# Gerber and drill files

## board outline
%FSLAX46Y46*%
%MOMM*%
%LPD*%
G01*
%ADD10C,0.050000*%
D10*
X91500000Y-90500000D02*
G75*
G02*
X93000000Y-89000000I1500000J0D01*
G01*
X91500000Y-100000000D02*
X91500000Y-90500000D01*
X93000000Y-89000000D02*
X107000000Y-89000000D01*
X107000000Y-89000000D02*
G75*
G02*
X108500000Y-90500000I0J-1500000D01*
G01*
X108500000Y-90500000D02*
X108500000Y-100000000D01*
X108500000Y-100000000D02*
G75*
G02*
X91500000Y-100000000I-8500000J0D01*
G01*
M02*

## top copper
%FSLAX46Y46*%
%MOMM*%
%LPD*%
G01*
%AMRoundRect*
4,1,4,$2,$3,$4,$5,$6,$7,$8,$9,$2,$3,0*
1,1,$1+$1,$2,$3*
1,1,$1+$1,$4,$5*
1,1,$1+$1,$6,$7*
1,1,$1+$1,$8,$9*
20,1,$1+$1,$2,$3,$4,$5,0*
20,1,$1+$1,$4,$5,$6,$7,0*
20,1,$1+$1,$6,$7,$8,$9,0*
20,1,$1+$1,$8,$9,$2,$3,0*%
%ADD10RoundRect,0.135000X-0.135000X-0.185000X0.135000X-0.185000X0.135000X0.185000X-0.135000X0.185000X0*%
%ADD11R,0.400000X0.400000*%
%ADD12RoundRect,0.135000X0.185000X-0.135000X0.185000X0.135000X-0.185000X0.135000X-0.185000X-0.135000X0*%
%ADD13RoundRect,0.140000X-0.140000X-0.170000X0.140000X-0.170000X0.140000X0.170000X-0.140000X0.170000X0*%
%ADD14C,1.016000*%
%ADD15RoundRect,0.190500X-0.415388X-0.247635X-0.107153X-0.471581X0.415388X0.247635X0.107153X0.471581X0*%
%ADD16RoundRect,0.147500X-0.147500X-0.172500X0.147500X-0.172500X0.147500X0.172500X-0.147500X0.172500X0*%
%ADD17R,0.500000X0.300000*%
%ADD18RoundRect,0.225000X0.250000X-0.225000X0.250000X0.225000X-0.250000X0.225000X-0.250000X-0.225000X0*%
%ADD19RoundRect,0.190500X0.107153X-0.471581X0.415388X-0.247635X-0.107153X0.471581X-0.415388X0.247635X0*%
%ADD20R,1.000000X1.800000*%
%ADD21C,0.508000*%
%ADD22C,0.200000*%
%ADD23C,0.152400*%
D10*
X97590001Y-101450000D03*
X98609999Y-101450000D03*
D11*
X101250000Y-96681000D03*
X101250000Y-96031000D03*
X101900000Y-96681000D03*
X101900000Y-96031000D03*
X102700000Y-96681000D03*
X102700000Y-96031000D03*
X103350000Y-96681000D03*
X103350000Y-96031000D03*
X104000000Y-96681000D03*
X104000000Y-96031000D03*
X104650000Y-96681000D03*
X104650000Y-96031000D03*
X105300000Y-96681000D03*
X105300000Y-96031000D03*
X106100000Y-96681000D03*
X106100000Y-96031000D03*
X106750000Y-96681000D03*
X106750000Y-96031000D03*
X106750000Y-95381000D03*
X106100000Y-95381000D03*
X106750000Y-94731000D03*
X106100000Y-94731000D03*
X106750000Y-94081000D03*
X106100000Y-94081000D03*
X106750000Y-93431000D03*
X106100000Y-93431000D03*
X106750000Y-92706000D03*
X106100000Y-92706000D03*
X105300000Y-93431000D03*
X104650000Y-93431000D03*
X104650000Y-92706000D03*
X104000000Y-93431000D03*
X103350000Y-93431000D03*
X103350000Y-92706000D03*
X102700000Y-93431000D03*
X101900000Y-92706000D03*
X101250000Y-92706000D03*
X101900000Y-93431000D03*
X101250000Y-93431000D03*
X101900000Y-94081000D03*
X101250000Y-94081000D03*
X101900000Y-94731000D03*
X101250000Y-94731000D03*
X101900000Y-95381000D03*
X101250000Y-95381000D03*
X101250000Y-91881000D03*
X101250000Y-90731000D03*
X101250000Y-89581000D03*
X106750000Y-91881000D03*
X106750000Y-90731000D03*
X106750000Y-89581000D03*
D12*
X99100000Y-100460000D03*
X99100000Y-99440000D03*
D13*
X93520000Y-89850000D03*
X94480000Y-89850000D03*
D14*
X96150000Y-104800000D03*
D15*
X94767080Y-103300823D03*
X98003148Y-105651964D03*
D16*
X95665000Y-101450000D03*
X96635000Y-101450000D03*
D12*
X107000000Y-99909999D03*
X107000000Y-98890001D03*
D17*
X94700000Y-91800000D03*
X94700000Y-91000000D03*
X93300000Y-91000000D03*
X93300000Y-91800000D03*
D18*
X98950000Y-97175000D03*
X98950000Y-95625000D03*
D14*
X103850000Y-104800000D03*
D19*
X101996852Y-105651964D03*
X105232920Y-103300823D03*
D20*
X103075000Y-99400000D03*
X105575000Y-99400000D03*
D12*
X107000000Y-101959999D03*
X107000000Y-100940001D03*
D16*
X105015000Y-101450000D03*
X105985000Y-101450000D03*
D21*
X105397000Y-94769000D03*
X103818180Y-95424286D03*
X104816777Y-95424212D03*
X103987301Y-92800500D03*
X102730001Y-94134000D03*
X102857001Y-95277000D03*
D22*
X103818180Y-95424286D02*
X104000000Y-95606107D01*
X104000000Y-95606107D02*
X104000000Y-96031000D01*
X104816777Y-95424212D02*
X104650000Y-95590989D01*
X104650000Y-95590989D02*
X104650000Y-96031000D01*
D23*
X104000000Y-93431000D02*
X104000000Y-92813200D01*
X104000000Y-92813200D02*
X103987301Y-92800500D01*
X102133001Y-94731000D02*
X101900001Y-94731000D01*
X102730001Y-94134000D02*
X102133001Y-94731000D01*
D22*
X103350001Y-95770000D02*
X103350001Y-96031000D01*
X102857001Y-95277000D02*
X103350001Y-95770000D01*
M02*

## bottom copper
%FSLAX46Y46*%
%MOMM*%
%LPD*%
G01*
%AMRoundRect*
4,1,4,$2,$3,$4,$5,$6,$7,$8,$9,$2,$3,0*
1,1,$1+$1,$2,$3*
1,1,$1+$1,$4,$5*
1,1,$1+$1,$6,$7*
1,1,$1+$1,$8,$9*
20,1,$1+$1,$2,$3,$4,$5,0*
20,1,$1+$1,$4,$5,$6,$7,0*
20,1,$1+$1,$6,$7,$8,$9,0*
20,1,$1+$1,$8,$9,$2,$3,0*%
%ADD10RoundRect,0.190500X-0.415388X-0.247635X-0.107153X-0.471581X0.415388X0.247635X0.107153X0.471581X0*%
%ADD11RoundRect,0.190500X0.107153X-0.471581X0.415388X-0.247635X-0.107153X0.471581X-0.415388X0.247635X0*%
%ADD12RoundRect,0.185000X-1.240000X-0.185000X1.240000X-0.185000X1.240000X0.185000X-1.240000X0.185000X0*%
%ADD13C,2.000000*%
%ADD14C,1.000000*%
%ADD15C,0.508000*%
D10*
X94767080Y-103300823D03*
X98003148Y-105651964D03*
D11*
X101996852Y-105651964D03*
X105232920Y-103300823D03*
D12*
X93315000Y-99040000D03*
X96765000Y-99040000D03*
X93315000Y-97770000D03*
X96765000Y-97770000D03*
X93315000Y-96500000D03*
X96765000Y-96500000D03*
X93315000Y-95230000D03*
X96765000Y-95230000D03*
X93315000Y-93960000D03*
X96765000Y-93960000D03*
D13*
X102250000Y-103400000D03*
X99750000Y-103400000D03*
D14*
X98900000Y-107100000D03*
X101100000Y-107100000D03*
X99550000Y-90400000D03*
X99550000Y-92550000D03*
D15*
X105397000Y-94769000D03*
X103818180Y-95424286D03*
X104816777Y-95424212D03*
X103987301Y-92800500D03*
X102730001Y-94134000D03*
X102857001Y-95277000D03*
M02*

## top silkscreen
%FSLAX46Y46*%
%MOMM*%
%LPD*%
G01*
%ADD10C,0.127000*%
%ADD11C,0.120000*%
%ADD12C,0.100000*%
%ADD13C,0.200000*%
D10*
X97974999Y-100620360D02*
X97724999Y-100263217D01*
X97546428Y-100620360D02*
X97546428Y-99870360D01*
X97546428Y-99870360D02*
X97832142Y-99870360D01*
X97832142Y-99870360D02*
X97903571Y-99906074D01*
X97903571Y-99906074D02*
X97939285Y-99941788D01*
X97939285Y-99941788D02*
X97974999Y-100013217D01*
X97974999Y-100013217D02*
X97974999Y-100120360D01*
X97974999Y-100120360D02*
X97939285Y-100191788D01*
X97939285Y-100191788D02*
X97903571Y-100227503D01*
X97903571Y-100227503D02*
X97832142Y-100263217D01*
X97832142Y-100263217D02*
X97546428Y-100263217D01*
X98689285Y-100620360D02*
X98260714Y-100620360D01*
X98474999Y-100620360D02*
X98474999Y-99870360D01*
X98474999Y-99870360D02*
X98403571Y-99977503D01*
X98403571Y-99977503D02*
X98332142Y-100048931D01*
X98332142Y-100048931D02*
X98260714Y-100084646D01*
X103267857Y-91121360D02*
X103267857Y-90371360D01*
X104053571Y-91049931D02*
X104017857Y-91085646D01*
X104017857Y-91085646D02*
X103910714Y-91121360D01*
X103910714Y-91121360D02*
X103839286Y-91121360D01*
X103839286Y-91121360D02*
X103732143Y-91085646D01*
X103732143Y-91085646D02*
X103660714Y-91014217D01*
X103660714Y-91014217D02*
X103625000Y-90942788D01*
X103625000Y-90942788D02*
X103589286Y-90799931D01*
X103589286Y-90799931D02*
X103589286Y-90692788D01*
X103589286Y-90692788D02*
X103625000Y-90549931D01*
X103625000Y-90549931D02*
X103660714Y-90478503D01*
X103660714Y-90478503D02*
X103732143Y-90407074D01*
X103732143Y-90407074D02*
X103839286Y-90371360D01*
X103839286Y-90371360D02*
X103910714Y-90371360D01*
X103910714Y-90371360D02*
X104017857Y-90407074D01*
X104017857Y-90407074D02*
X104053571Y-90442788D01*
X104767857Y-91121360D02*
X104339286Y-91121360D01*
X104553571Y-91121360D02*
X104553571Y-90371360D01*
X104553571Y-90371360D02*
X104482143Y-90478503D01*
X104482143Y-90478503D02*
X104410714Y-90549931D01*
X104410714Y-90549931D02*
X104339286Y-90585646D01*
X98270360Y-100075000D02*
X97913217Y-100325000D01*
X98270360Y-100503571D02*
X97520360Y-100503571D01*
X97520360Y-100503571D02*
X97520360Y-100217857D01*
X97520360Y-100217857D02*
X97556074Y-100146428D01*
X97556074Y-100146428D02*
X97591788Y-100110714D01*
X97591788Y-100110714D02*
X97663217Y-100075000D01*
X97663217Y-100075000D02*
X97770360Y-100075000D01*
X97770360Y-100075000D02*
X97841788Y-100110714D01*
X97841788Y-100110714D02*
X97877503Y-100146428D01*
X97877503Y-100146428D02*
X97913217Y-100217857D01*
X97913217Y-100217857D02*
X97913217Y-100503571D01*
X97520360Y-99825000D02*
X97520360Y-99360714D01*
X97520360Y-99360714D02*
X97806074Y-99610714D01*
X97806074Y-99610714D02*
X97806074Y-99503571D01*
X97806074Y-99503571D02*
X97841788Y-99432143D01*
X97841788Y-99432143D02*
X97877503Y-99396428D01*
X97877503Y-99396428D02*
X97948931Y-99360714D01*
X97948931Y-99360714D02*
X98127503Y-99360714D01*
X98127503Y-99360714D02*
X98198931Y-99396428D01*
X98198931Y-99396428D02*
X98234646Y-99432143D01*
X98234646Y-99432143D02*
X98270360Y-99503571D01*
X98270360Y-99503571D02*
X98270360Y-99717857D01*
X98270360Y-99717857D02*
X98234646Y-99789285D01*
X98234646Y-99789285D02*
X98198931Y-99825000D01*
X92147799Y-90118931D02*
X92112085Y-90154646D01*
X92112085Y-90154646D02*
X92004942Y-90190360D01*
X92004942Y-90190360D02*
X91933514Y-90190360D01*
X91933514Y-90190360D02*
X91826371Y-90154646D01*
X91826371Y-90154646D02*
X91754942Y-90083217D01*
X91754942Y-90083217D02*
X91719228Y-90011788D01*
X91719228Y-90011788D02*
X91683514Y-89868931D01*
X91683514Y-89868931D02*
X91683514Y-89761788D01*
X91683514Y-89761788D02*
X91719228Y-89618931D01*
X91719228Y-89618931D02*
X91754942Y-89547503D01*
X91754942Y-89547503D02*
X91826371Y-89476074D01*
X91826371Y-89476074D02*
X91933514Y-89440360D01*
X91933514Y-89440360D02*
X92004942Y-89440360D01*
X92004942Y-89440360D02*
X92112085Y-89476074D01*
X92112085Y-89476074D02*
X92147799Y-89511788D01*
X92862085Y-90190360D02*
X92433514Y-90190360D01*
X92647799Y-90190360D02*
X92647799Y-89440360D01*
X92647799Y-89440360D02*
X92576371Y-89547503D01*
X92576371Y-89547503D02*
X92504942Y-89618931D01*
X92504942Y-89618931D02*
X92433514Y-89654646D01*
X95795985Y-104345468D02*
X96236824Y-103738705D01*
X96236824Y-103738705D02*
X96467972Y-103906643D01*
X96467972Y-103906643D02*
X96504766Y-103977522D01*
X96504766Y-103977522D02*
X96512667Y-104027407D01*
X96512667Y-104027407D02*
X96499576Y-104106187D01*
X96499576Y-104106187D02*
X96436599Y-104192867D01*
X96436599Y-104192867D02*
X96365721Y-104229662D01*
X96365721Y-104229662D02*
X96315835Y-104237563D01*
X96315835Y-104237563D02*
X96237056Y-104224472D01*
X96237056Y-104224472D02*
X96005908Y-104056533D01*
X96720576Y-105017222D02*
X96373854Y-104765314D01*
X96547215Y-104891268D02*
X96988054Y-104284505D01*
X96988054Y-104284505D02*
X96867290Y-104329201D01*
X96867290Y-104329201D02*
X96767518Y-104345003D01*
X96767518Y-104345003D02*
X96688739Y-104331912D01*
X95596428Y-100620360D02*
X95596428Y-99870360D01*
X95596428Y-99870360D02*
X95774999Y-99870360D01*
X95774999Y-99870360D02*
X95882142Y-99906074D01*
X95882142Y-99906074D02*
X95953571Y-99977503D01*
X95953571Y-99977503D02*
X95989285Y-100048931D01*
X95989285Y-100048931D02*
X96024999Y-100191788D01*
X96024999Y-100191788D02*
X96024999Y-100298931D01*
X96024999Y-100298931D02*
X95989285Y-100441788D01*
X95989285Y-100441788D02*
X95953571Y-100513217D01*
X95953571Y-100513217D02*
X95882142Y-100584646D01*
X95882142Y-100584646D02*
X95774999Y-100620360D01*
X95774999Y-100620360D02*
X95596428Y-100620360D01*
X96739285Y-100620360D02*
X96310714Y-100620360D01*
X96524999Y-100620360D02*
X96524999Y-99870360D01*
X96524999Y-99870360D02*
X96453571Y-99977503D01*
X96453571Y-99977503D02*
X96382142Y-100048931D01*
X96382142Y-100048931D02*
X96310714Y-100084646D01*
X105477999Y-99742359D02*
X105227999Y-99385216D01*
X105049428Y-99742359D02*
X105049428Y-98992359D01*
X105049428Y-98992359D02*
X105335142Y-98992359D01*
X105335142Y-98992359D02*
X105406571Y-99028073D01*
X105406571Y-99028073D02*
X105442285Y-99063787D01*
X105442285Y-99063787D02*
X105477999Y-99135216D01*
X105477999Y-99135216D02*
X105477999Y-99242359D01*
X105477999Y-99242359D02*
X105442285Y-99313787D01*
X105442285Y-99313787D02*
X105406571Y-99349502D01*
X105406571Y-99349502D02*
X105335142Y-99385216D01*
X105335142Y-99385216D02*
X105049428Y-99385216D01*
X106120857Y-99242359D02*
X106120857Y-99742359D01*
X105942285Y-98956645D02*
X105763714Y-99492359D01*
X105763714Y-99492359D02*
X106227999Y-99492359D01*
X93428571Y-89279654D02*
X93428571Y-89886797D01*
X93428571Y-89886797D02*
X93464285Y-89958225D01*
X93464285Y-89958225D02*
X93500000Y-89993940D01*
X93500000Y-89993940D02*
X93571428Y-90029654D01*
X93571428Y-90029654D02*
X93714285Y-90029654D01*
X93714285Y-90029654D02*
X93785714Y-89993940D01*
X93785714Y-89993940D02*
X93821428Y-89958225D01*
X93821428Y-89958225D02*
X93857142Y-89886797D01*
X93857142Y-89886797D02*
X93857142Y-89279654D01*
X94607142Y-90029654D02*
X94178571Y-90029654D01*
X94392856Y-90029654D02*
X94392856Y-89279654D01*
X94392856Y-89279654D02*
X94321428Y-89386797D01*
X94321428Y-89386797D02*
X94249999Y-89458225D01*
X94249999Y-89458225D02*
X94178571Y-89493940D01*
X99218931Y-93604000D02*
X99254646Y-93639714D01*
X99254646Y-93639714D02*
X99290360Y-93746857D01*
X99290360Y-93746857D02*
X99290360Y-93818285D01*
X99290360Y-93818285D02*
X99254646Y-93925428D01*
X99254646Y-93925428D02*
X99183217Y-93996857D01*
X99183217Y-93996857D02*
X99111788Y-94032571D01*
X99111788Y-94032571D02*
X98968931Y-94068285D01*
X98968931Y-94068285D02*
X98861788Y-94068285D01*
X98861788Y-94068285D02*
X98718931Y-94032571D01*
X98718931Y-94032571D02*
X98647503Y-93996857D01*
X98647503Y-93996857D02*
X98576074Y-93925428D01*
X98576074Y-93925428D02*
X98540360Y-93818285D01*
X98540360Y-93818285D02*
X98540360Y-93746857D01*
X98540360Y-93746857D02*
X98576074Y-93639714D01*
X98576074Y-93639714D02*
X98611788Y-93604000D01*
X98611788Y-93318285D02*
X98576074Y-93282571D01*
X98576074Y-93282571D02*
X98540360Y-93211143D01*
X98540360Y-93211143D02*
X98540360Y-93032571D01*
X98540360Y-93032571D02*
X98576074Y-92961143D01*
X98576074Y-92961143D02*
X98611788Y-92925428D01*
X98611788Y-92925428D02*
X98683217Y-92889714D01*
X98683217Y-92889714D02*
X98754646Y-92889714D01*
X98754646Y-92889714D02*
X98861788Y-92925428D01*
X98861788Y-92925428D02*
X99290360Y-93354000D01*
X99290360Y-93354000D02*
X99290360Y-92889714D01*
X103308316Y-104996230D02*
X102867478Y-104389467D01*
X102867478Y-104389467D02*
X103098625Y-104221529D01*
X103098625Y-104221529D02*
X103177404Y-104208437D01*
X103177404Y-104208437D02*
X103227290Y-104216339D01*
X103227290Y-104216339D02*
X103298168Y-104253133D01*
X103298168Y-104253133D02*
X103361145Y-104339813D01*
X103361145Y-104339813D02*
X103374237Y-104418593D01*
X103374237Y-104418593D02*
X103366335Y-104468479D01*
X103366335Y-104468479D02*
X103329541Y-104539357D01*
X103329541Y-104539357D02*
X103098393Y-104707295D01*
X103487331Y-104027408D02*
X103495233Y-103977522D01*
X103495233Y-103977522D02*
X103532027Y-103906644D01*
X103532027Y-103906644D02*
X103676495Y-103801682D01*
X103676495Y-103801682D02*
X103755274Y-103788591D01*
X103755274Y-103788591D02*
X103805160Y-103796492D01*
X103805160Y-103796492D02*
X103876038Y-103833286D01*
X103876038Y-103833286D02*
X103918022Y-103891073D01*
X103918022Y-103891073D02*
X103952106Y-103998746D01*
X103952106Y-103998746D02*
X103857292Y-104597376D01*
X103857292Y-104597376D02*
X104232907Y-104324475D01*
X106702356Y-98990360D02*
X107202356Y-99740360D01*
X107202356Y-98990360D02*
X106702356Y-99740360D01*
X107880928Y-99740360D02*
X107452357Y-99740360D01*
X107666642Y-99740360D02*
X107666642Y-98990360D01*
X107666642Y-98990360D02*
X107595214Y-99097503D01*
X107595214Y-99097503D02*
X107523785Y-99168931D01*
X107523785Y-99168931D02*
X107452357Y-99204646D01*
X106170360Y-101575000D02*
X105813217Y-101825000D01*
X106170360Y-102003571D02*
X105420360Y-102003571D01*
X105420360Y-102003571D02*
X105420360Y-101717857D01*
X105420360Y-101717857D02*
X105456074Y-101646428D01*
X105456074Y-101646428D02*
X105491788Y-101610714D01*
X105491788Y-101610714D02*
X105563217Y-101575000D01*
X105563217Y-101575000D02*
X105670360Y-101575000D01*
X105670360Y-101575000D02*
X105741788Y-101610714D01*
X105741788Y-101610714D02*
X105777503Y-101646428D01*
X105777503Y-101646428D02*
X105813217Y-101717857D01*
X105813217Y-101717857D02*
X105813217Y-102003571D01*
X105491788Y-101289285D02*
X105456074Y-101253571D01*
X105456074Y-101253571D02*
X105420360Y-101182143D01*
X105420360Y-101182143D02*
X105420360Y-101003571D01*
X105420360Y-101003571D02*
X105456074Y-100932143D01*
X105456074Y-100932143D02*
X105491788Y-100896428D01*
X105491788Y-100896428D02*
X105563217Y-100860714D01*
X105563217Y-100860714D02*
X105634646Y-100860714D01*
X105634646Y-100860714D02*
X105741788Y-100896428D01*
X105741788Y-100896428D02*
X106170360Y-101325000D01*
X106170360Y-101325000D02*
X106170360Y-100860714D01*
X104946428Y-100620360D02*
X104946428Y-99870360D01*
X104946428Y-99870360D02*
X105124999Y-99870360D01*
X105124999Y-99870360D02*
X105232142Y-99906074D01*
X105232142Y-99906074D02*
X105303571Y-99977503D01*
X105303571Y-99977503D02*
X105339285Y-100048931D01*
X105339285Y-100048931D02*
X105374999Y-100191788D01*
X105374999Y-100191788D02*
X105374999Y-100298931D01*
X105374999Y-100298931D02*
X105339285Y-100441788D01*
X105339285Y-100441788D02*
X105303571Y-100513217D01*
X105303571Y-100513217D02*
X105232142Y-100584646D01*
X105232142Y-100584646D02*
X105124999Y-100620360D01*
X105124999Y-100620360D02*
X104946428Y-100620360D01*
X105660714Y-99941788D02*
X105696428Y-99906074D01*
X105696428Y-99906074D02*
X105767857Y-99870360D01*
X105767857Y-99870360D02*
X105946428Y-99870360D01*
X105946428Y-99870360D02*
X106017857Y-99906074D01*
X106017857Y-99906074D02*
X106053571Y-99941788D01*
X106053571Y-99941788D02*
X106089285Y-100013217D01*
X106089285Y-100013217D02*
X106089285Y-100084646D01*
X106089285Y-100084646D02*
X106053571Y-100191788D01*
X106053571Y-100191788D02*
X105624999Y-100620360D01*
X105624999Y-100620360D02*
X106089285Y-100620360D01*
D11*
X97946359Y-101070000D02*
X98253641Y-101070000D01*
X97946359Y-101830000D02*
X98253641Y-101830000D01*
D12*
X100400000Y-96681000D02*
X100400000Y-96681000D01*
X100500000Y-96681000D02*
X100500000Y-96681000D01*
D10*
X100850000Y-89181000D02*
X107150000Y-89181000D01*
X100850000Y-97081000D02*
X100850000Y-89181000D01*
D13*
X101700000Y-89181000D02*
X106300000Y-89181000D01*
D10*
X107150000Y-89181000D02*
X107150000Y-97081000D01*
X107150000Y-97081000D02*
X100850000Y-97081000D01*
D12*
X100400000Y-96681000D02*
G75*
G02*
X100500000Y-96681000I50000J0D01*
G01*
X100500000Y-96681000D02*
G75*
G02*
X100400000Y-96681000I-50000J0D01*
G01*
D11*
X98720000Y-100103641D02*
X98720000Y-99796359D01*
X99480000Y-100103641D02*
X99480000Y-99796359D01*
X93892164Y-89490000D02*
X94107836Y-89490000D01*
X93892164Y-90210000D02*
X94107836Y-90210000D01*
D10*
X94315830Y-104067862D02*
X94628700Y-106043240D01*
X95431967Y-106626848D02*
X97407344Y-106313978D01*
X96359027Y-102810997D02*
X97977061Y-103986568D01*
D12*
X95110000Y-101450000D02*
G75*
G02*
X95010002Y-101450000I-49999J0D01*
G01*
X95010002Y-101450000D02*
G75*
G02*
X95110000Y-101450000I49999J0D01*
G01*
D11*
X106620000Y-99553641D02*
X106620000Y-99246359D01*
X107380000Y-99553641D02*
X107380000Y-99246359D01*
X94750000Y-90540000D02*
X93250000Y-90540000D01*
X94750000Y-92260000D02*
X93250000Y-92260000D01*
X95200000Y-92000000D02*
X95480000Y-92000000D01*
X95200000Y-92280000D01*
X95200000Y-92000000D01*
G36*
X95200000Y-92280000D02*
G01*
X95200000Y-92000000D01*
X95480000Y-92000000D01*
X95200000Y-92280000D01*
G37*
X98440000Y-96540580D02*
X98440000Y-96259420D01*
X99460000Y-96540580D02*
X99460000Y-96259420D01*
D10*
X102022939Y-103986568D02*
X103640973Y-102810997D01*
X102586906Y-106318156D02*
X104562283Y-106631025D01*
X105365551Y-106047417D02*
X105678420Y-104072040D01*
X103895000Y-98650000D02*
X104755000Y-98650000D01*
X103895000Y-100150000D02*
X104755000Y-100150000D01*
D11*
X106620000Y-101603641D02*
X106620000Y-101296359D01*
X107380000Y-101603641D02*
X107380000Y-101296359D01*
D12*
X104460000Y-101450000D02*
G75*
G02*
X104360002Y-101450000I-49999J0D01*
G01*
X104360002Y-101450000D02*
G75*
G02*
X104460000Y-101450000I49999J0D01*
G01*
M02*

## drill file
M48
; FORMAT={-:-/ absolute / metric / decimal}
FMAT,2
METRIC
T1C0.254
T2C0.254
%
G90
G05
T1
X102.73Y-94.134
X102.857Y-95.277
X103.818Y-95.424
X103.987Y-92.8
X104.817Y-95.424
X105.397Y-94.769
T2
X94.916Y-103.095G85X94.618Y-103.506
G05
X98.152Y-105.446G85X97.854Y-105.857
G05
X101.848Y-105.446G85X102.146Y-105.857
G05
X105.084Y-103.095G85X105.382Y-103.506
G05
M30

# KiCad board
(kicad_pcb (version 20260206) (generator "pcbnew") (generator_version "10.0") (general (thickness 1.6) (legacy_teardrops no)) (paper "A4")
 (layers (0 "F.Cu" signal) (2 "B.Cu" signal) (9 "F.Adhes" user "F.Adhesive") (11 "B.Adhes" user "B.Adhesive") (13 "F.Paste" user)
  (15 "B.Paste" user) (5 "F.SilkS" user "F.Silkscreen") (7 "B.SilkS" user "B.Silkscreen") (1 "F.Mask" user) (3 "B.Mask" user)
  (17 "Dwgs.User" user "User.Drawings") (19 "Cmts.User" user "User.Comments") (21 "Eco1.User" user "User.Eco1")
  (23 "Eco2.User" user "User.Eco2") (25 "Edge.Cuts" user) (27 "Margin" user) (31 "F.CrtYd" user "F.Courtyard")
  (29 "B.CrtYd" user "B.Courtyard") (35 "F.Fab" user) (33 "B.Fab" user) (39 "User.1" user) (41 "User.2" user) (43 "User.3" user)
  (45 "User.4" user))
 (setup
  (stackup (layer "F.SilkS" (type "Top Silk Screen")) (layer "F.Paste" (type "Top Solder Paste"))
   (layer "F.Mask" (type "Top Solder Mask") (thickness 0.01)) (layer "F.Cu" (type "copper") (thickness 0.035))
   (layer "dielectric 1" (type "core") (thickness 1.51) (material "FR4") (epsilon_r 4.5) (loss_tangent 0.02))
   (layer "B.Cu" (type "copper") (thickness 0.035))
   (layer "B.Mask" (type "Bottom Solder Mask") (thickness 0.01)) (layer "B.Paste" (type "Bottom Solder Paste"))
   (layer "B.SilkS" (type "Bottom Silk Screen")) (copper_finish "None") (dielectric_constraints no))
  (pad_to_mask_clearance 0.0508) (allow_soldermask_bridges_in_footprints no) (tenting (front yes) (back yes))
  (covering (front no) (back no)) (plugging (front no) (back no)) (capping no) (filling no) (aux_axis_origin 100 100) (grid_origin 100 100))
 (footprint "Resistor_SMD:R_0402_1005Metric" (layer "F.Cu") (at 98.1 101.45)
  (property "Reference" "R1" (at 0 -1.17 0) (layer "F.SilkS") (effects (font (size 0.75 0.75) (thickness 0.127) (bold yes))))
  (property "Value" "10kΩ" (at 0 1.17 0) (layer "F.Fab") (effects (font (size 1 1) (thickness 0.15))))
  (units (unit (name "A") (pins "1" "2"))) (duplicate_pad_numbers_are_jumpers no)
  (fp_line (start -0.153641 -0.38) (end 0.153641 -0.38) (stroke (width 0.12) (type solid)) (layer "F.SilkS"))
  (fp_line (start -0.153641 0.38) (end 0.153641 0.38) (stroke (width 0.12) (type solid)) (layer "F.SilkS"))
  (pad "1" smd roundrect (at -0.509999 0) (size 0.54 0.64) (layers "F.Cu" "F.Mask" "F.Paste") (roundrect_rratio 0.25) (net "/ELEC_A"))
  (pad "2" smd roundrect (at 0.509999 0) (size 0.54 0.64) (layers "F.Cu" "F.Mask" "F.Paste") (roundrect_rratio 0.25) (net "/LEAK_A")))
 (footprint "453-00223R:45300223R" (layer "F.Cu") (at 104 89.181 90)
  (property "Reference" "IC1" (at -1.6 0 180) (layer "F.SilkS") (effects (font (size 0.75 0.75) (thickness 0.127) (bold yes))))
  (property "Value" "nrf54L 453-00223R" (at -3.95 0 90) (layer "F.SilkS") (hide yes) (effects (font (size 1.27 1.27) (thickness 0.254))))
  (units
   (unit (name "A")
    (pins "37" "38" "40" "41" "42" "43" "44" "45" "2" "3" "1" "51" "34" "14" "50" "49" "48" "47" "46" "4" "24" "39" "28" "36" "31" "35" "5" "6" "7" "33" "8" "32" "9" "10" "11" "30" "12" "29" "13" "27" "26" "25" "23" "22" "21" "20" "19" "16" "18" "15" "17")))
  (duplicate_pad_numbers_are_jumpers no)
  (fp_line (start -7.5 -3.6) (end -7.5 -3.6) (stroke (width 0.1) (type solid)) (layer "F.SilkS"))
  (fp_line (start -7.5 -3.5) (end -7.5 -3.5) (stroke (width 0.1) (type solid)) (layer "F.SilkS"))
  (fp_line (start 0 -3.15) (end 0 3.15) (stroke (width 0.127) (type solid)) (layer "F.SilkS"))
  (fp_line (start -7.9 -3.15) (end 0 -3.15) (stroke (width 0.127) (type solid)) (layer "F.SilkS"))
  (fp_line (start 0 -2.3) (end 0 2.3) (stroke (width 0.2) (type solid)) (layer "F.SilkS"))
  (fp_line (start 0 3.15) (end -7.9 3.15) (stroke (width 0.127) (type solid)) (layer "F.SilkS"))
  (fp_line (start -7.9 3.15) (end -7.9 -3.15) (stroke (width 0.127) (type solid)) (layer "F.SilkS"))
  (fp_arc (start -7.5 -3.6) (mid -7.45 -3.55) (end -7.5 -3.5) (stroke (width 0.1) (type solid)) (layer "F.SilkS"))
  (fp_arc (start -7.5 -3.5) (mid -7.55 -3.55) (end -7.5 -3.6) (stroke (width 0.1) (type solid)) (layer "F.SilkS"))
  (pad "1" smd rect (at -7.5 -2.75 180) (size 0.4 0.4) (layers "F.Cu" "F.Mask" "F.Paste") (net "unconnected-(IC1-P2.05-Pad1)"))
  (pad "2" smd rect (at -6.85 -2.75 180) (size 0.4 0.4) (layers "F.Cu" "F.Mask" "F.Paste") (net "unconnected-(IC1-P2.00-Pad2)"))
  (pad "3" smd rect (at -7.5 -2.1 180) (size 0.4 0.4) (layers "F.Cu" "F.Mask" "F.Paste") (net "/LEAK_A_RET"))
  (pad "4" smd rect (at -6.85 -2.1 180) (size 0.4 0.4) (layers "F.Cu" "F.Mask" "F.Paste") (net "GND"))
  (pad "5" smd rect (at -7.5 -1.3 180) (size 0.4 0.4) (layers "F.Cu" "F.Mask" "F.Paste") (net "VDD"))
  (pad "6" smd rect (at -6.85 -1.3 180) (size 0.4 0.4) (layers "F.Cu" "F.Mask" "F.Paste") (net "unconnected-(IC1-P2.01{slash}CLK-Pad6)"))
  (pad "7" smd rect (at -7.5 -0.65 180) (size 0.4 0.4) (layers "F.Cu" "F.Mask" "F.Paste") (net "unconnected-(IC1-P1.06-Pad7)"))
  (pad "8" smd rect (at -6.85 -0.65 180) (size 0.4 0.4) (layers "F.Cu" "F.Mask" "F.Paste") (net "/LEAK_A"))
  (pad "9" smd rect (at -7.5 0 180) (size 0.4 0.4) (layers "F.Cu" "F.Mask" "F.Paste")
   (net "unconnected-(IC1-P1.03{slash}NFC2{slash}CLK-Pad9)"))
  (pad "10" smd rect (at -6.85 0 180) (size 0.4 0.4) (layers "F.Cu" "F.Mask" "F.Paste") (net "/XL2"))
  (pad "11" smd rect (at -7.5 0.65 180) (size 0.4 0.4) (layers "F.Cu" "F.Mask" "F.Paste") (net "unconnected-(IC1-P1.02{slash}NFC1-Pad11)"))
  (pad "12" smd rect (at -6.85 0.65 180) (size 0.4 0.4) (layers "F.Cu" "F.Mask" "F.Paste") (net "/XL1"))
  (pad "13" smd rect (at -7.5 1.3 180) (size 0.4 0.4) (layers "F.Cu" "F.Mask" "F.Paste") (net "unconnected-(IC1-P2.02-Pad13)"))
  (pad "14" smd rect (at -6.85 1.3 180) (size 0.4 0.4) (layers "F.Cu" "F.Mask" "F.Paste") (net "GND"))
  (pad "15" smd rect (at -7.5 2.1 180) (size 0.4 0.4) (layers "F.Cu" "F.Mask" "F.Paste") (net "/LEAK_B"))
  (pad "16" smd rect (at -6.85 2.1 180) (size 0.4 0.4) (layers "F.Cu" "F.Mask" "F.Paste") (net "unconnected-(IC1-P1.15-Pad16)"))
  (pad "17" smd rect (at -7.5 2.75 180) (size 0.4 0.4) (layers "F.Cu" "F.Mask" "F.Paste") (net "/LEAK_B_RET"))
  (pad "18" smd rect (at -6.85 2.75 180) (size 0.4 0.4) (layers "F.Cu" "F.Mask" "F.Paste") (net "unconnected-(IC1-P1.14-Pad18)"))
  (pad "19" smd rect (at -6.2 2.75 180) (size 0.4 0.4) (layers "F.Cu" "F.Mask" "F.Paste") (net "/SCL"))
  (pad "20" smd rect (at -6.2 2.1 180) (size 0.4 0.4) (layers "F.Cu" "F.Mask" "F.Paste") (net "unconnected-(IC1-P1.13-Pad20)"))
  (pad "21" smd rect (at -5.55 2.75 180) (size 0.4 0.4) (layers "F.Cu" "F.Mask" "F.Paste") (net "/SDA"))
  (pad "22" smd rect (at -5.55 2.1 180) (size 0.4 0.4) (layers "F.Cu" "F.Mask" "F.Paste") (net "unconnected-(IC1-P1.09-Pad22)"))
  (pad "23" smd rect (at -4.9 2.75 180) (size 0.4 0.4) (layers "F.Cu" "F.Mask" "F.Paste")
   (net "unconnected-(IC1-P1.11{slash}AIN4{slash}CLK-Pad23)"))
  (pad "24" smd rect (at -4.9 2.1 180) (size 0.4 0.4) (layers "F.Cu" "F.Mask" "F.Paste") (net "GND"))
  (pad "25" smd rect (at -4.25 2.75 180) (size 0.4 0.4) (layers "F.Cu" "F.Mask" "F.Paste") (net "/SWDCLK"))
  (pad "26" smd rect (at -4.25 2.1 180) (size 0.4 0.4) (layers "F.Cu" "F.Mask" "F.Paste") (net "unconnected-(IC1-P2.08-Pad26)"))
  (pad "27" smd rect (at -3.525 2.75 180) (size 0.4 0.4) (layers "F.Cu" "F.Mask" "F.Paste") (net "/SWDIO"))
  (pad "28" smd rect (at -3.525 2.1 180) (size 0.4 0.4) (layers "F.Cu" "F.Mask" "F.Paste") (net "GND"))
  (pad "29" smd rect (at -4.25 1.3 180) (size 0.4 0.4) (layers "F.Cu" "F.Mask" "F.Paste") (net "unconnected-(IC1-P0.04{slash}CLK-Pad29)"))
  (pad "30" smd rect (at -4.25 0.65 180) (size 0.4 0.4) (layers "F.Cu" "F.Mask" "F.Paste") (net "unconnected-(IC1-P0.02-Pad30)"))
  (pad "31" smd rect (at -3.525 0.65 180) (size 0.4 0.4) (layers "F.Cu" "F.Mask" "F.Paste") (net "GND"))
  (pad "32" smd rect (at -4.25 0 180) (size 0.4 0.4) (layers "F.Cu" "F.Mask" "F.Paste") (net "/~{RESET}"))
  (pad "33" smd rect (at -4.25 -0.65 180) (size 0.4 0.4) (layers "F.Cu" "F.Mask" "F.Paste") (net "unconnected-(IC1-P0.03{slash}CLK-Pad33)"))
  (pad "34" smd rect (at -3.525 -0.65 180) (size 0.4 0.4) (layers "F.Cu" "F.Mask" "F.Paste") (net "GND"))
  (pad "35" smd rect (at -4.25 -1.3 180) (size 0.4 0.4) (layers "F.Cu" "F.Mask" "F.Paste") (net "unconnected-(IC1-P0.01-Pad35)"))
  (pad "36" smd rect (at -3.525 -2.1 180) (size 0.4 0.4) (layers "F.Cu" "F.Mask" "F.Paste") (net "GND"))
  (pad "37" smd rect (at -3.525 -2.75 180) (size 0.4 0.4) (layers "F.Cu" "F.Mask" "F.Paste") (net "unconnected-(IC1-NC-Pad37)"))
  (pad "38" smd rect (at -4.25 -2.1 180) (size 0.4 0.4) (layers "F.Cu" "F.Mask" "F.Paste") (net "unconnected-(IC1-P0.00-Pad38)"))
  (pad "39" smd rect (at -4.25 -2.75 180) (size 0.4 0.4) (layers "F.Cu" "F.Mask" "F.Paste") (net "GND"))
  (pad "40" smd rect (at -4.9 -2.1 180) (size 0.4 0.4) (layers "F.Cu" "F.Mask" "F.Paste") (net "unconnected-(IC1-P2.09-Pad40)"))
  (pad "41" smd rect (at -4.9 -2.75 180) (size 0.4 0.4) (layers "F.Cu" "F.Mask" "F.Paste") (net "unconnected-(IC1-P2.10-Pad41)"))
  (pad "42" smd rect (at -5.55 -2.1 180) (size 0.4 0.4) (layers "F.Cu" "F.Mask" "F.Paste") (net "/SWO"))
  (pad "43" smd rect (at -5.55 -2.75 180) (size 0.4 0.4) (layers "F.Cu" "F.Mask" "F.Paste") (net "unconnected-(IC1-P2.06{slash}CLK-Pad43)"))
  (pad "44" smd rect (at -6.2 -2.1 180) (size 0.4 0.4) (layers "F.Cu" "F.Mask" "F.Paste") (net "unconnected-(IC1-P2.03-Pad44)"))
  (pad "45" smd rect (at -6.2 -2.75 180) (size 0.4 0.4) (layers "F.Cu" "F.Mask" "F.Paste") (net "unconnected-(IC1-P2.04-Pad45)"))
  (pad "46" smd rect (at -2.7 -2.75 180) (size 0.4 0.4) (layers "F.Cu" "F.Mask" "F.Paste") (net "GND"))
  (pad "47" smd rect (at -1.55 -2.75 180) (size 0.4 0.4) (layers "F.Cu" "F.Mask" "F.Paste") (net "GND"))
  (pad "48" smd rect (at -0.4 -2.75 180) (size 0.4 0.4) (layers "F.Cu" "F.Mask" "F.Paste") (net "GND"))
  (pad "49" smd rect (at -2.7 2.75 180) (size 0.4 0.4) (layers "F.Cu" "F.Mask" "F.Paste") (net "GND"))
  (pad "50" smd rect (at -1.55 2.75 180) (size 0.4 0.4) (layers "F.Cu" "F.Mask" "F.Paste") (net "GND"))
  (pad "51" smd rect (at -0.4 2.75 180) (size 0.4 0.4) (layers "F.Cu" "F.Mask" "F.Paste") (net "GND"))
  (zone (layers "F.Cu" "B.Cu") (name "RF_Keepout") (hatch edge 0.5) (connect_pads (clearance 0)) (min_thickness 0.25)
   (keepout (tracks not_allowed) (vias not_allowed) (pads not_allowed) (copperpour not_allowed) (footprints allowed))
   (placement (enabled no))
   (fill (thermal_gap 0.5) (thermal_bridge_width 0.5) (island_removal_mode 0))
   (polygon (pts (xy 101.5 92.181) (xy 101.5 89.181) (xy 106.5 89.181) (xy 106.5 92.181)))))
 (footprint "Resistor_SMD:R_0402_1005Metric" (layer "F.Cu") (at 99.1 99.95 90)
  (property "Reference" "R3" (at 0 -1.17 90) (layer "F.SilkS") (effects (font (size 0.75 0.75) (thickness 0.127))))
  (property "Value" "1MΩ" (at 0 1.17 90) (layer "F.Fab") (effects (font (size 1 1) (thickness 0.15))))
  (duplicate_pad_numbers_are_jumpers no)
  (fp_line (start -0.153641 -0.38) (end 0.153641 -0.38) (stroke (width 0.12) (type solid)) (layer "F.SilkS"))
  (fp_line (start -0.153641 0.38) (end 0.153641 0.38) (stroke (width 0.12) (type solid)) (layer "F.SilkS"))
  (pad "1" smd roundrect (at -0.51 0 90) (size 0.54 0.64) (layers "F.Cu" "F.Mask" "F.Paste") (roundrect_rratio 0.25) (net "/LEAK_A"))
  (pad "2" smd roundrect (at 0.51 0 90) (size 0.54 0.64) (layers "F.Cu" "F.Mask" "F.Paste") (roundrect_rratio 0.25) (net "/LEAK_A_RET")))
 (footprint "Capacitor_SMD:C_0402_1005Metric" (layer "F.Cu") (at 94 89.85)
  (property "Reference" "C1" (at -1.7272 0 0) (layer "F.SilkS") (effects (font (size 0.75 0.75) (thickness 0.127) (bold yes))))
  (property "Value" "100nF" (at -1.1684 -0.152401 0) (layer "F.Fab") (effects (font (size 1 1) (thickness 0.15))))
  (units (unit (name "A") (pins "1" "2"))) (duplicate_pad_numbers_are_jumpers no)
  (fp_line (start -0.107836 -0.36) (end 0.107836 -0.36) (stroke (width 0.12) (type solid)) (layer "F.SilkS"))
  (fp_line (start -0.107836 0.36) (end 0.107836 0.36) (stroke (width 0.12) (type solid)) (layer "F.SilkS"))
  (pad "1" smd roundrect (at -0.48 0) (size 0.56 0.62) (layers "F.Cu" "F.Mask" "F.Paste") (roundrect_rratio 0.25) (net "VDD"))
  (pad "2" smd roundrect (at 0.48 0) (size 0.56 0.62) (layers "F.Cu" "F.Mask" "F.Paste") (roundrect_rratio 0.25) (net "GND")))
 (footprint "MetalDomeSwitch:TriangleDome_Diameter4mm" (layer "F.Cu") (at 96.15 104.8 -36)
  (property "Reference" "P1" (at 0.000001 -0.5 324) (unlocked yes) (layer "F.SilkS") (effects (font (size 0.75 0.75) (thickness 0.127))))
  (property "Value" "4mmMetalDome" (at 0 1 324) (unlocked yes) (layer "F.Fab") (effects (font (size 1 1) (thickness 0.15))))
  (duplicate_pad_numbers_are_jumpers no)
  (fp_line (start -1.914215 0.485786) (end -0.499999 1.9) (stroke (width 0.127) (type solid)) (layer "F.SilkS"))
  (fp_line (start 0.492893 1.9) (end 1.907107 0.485786) (stroke (width 0.127) (type solid)) (layer "F.SilkS"))
  (fp_line (start -1 -1.732) (end 1 -1.732) (stroke (width 0.127) (type default)) (layer "F.SilkS"))
  (pad "1" smd circle (at 0 0 324) (size 1.016 1.016) (layers "F.Cu" "F.Mask" "F.Paste") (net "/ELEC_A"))
  (pad "2" thru_hole roundrect (at -2 -0.4 324) (size 0.762 1.27) (drill oval 0.254 0.762) (layers "*.Cu" "*.Mask")
   (remove_unused_layers no) (roundrect_rratio 0.25) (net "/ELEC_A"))
  (pad "2" thru_hole roundrect (at 2 -0.4 324) (size 0.762 1.27) (drill oval 0.254 0.762) (layers "*.Cu" "*.Mask") (remove_unused_layers no)
   (roundrect_rratio 0.25) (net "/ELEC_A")))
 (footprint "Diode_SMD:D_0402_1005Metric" (layer "F.Cu") (at 96.15 101.45)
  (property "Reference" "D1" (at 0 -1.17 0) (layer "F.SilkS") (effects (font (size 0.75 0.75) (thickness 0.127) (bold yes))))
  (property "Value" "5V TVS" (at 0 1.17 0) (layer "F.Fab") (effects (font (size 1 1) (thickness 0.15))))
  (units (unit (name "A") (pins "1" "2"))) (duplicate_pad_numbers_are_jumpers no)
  (fp_circle (center -1.089999 0) (end -1.04 0) (stroke (width 0.1) (type solid)) (fill no) (layer "F.SilkS"))
  (pad "1" smd roundrect (at -0.485 0) (size 0.59 0.64) (layers "F.Cu" "F.Mask" "F.Paste") (roundrect_rratio 0.25) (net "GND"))
  (pad "2" smd roundrect (at 0.485 0) (size 0.59 0.64) (layers "F.Cu" "F.Mask" "F.Paste") (roundrect_rratio 0.25) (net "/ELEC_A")))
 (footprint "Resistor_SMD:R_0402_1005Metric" (layer "F.Cu") (at 107 99.4 90)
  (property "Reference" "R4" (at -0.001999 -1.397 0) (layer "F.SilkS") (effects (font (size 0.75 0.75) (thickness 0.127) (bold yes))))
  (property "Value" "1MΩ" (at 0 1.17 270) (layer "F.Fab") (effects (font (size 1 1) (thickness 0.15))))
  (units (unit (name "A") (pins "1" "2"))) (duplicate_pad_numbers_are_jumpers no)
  (fp_line (start -0.153641 -0.38) (end 0.153641 -0.38) (stroke (width 0.12) (type solid)) (layer "F.SilkS"))
  (fp_line (start -0.153641 0.38) (end 0.153641 0.38) (stroke (width 0.12) (type solid)) (layer "F.SilkS"))
  (pad "1" smd roundrect (at -0.509999 0 90) (size 0.54 0.64) (layers "F.Cu" "F.Mask" "F.Paste") (roundrect_rratio 0.25) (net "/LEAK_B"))
  (pad "2" smd roundrect (at 0.509999 0 90) (size 0.54 0.64) (layers "F.Cu" "F.Mask" "F.Paste") (roundrect_rratio 0.25) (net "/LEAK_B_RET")))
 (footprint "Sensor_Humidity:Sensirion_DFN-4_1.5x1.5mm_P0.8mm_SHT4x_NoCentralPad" (layer "F.Cu") (at 94 91.4 180)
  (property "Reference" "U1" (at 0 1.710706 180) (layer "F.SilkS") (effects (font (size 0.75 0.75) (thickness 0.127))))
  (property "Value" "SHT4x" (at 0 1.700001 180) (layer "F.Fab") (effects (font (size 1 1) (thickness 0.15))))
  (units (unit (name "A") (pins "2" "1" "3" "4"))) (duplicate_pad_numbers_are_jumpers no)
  (fp_line (start -0.75 0.86) (end 0.75 0.86) (stroke (width 0.12) (type solid)) (layer "F.SilkS"))
  (fp_line (start -0.75 -0.86) (end 0.75 -0.86) (stroke (width 0.12) (type solid)) (layer "F.SilkS"))
  (fp_poly
   (pts (xy -1.2 -0.6) (xy -1.48 -0.6) (xy -1.2 -0.88) (xy -1.2 -0.6)) (stroke (width 0.12) (type solid)) (fill yes) (layer "F.SilkS"))
  (pad "1" smd rect (at -0.7 -0.4 180) (size 0.5 0.3) (layers "F.Cu" "F.Mask" "F.Paste") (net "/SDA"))
  (pad "2" smd rect (at -0.7 0.4 180) (size 0.5 0.3) (layers "F.Cu" "F.Mask" "F.Paste") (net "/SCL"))
  (pad "3" smd rect (at 0.7 0.4 180) (size 0.5 0.3) (layers "F.Cu" "F.Mask" "F.Paste") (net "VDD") (clearance 0.1524))
  (pad "4" smd rect (at 0.7 -0.4 180) (size 0.5 0.3) (layers "F.Cu" "F.Mask" "F.Paste") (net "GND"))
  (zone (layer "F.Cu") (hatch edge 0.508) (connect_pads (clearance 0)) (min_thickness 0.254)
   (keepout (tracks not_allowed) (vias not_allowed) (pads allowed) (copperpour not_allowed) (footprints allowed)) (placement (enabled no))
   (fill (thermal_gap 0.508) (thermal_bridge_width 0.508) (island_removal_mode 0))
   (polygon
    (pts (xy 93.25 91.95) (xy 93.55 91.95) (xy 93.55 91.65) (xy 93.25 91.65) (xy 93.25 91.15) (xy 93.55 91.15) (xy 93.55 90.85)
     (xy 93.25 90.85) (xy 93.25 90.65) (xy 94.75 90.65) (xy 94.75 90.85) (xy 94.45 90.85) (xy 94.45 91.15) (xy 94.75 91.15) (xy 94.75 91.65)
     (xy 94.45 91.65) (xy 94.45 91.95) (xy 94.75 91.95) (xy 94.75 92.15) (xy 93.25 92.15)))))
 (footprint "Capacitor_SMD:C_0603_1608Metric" (layer "F.Cu") (at 98.95 96.4 90)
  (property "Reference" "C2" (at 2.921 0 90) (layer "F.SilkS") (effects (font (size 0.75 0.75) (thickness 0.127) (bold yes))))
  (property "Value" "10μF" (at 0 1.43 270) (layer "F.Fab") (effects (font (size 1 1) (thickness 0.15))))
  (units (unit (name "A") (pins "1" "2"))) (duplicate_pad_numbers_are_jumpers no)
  (fp_line (start -0.14058 -0.51) (end 0.14058 -0.51) (stroke (width 0.12) (type solid)) (layer "F.SilkS"))
  (fp_line (start -0.14058 0.51) (end 0.14058 0.51) (stroke (width 0.12) (type solid)) (layer "F.SilkS"))
  (pad "1" smd roundrect (at -0.775 0 90) (size 0.9 0.95) (layers "F.Cu" "F.Mask" "F.Paste") (roundrect_rratio 0.25) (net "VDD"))
  (pad "2" smd roundrect (at 0.775 0 90) (size 0.9 0.95) (layers "F.Cu" "F.Mask" "F.Paste") (roundrect_rratio 0.25) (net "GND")))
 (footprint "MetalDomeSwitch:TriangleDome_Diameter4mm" (layer "F.Cu") (at 103.85 104.8 36)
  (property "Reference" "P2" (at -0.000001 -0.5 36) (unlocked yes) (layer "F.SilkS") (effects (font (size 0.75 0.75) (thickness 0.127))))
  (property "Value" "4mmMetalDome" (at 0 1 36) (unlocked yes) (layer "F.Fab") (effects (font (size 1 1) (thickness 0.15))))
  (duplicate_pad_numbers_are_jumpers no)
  (fp_line (start -1 -1.732) (end 1 -1.732) (stroke (width 0.127) (type default)) (layer "F.SilkS"))
  (fp_line (start -1.914214 0.485786) (end -0.5 1.9) (stroke (width 0.127) (type solid)) (layer "F.SilkS"))
  (fp_line (start 0.492893 1.9) (end 1.907107 0.485786) (stroke (width 0.127) (type solid)) (layer "F.SilkS"))
  (pad "1" smd circle (at 0 0 36) (size 1.016 1.016) (layers "F.Cu" "F.Mask" "F.Paste") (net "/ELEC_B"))
  (pad "2" thru_hole roundrect (at -2 -0.4 36) (size 0.762 1.27) (drill oval 0.254 0.762) (layers "*.Cu" "*.Mask") (remove_unused_layers no)
   (roundrect_rratio 0.25) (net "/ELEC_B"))
  (pad "2" thru_hole roundrect (at 2 -0.4 36) (size 0.762 1.27) (drill oval 0.254 0.762) (layers "*.Cu" "*.Mask") (remove_unused_layers no)
   (roundrect_rratio 0.25) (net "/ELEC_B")))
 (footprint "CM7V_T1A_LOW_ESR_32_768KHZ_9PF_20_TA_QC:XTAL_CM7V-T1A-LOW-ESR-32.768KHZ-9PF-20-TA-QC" (layer "F.Cu") (at 104.325 99.4)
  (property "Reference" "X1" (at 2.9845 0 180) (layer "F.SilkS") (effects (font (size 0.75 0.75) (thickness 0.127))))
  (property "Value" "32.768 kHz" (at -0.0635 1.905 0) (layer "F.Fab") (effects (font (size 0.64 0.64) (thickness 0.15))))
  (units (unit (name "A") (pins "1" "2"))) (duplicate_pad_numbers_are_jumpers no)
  (fp_line (start -0.43 -0.75) (end 0.43 -0.75) (stroke (width 0.127) (type solid)) (layer "F.SilkS"))
  (fp_line (start -0.43 0.75) (end 0.43 0.75) (stroke (width 0.127) (type solid)) (layer "F.SilkS"))
  (pad "1" smd rect (at -1.25 0) (size 1 1.8) (layers "F.Cu" "F.Mask" "F.Paste") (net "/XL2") (solder_mask_margin 0.102))
  (pad "2" smd rect (at 1.25 0) (size 1 1.8) (layers "F.Cu" "F.Mask" "F.Paste") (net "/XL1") (solder_mask_margin 0.102)))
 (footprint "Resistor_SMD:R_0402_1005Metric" (layer "F.Cu") (at 107 101.45 90)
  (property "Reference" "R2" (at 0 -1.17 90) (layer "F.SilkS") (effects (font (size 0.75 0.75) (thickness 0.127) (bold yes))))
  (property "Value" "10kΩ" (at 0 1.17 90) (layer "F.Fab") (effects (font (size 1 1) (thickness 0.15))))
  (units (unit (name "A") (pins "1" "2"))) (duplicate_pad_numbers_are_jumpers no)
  (fp_line (start -0.153641 -0.38) (end 0.153641 -0.38) (stroke (width 0.12) (type solid)) (layer "F.SilkS"))
  (fp_line (start -0.153641 0.38) (end 0.153641 0.38) (stroke (width 0.12) (type solid)) (layer "F.SilkS"))
  (pad "1" smd roundrect (at -0.509999 0 90) (size 0.54 0.64) (layers "F.Cu" "F.Mask" "F.Paste") (roundrect_rratio 0.25) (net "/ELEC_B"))
  (pad "2" smd roundrect (at 0.509999 0 90) (size 0.54 0.64) (layers "F.Cu" "F.Mask" "F.Paste") (roundrect_rratio 0.25) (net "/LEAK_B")))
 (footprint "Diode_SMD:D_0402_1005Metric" (layer "F.Cu") (at 105.5 101.45)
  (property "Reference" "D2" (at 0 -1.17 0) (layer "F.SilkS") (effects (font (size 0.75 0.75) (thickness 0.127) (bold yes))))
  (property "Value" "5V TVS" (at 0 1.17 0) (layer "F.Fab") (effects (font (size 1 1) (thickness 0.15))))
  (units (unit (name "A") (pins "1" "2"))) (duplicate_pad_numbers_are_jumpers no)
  (fp_circle (center -1.089999 0) (end -1.04 0) (stroke (width 0.1) (type solid)) (fill no) (layer "F.SilkS"))
  (pad "1" smd roundrect (at -0.485 0) (size 0.59 0.64) (layers "F.Cu" "F.Mask" "F.Paste") (roundrect_rratio 0.25) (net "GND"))
  (pad "2" smd roundrect (at 0.485 0) (size 0.59 0.64) (layers "F.Cu" "F.Mask" "F.Paste") (roundrect_rratio 0.25) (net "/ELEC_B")))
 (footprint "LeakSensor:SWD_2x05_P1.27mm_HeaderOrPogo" (layer "B.Cu") (at 95.04 96.5)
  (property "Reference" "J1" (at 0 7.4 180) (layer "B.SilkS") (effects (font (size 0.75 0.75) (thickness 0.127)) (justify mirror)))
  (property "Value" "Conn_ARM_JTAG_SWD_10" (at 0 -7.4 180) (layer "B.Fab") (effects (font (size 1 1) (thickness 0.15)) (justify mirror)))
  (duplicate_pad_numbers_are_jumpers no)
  (pad "1" smd roundrect (at -1.725 2.54) (size 2.85 0.74) (layers "B.Cu" "B.Mask") (roundrect_rratio 0.25) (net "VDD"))
  (pad "2" smd roundrect (at 1.725 2.54) (size 2.85 0.74) (layers "B.Cu" "B.Mask") (roundrect_rratio 0.25) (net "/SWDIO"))
  (pad "3" smd roundrect (at -1.725 1.27) (size 2.85 0.74) (layers "B.Cu" "B.Mask") (roundrect_rratio 0.25) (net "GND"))
  (pad "4" smd roundrect (at 1.725 1.27) (size 2.85 0.74) (layers "B.Cu" "B.Mask") (roundrect_rratio 0.25) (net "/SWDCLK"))
  (pad "5" smd roundrect (at -1.725 0) (size 2.85 0.74) (layers "B.Cu" "B.Mask") (roundrect_rratio 0.25) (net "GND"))
  (pad "6" smd roundrect (at 1.725 0) (size 2.85 0.74) (layers "B.Cu" "B.Mask") (roundrect_rratio 0.25) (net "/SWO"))
  (pad "7" smd roundrect (at -1.725 -1.27) (size 2.85 0.74) (layers "B.Cu" "B.Mask") (roundrect_rratio 0.25)
   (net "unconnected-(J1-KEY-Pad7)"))
  (pad "8" smd roundrect (at 1.725 -1.27) (size 2.85 0.74) (layers "B.Cu" "B.Mask") (roundrect_rratio 0.25)
   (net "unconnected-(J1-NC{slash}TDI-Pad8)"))
  (pad "9" smd roundrect (at -1.725 -2.54) (size 2.85 0.74) (layers "B.Cu" "B.Mask") (roundrect_rratio 0.25) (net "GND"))
  (pad "10" smd roundrect (at 1.725 -2.54) (size 2.85 0.74) (layers "B.Cu" "B.Mask") (roundrect_rratio 0.25) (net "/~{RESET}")))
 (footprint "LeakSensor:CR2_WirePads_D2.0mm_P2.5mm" (layer "B.Cu") (at 102.25 103.4 90)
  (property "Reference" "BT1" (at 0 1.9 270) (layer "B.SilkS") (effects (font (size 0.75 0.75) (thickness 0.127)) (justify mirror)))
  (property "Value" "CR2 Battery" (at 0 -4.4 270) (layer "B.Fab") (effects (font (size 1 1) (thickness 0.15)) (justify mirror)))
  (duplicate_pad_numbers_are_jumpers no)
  (pad "1" smd circle (at 0 0 90) (size 2 2) (layers "B.Cu" "B.Mask") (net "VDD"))
  (pad "2" smd circle (at 0 -2.5 90) (size 2 2) (layers "B.Cu" "B.Mask") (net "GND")))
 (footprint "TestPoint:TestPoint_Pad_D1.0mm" (layer "B.Cu") (at 98.9 107.1)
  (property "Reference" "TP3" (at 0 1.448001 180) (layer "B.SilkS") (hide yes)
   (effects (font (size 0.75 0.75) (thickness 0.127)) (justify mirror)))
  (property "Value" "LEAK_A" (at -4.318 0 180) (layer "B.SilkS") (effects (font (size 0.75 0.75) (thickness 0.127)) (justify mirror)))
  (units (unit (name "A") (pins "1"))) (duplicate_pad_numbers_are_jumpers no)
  (pad "1" smd circle (at 0 0) (size 1 1) (layers "B.Cu" "B.Mask") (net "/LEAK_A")))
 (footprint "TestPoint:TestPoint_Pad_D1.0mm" (layer "B.Cu") (at 101.1 107.1)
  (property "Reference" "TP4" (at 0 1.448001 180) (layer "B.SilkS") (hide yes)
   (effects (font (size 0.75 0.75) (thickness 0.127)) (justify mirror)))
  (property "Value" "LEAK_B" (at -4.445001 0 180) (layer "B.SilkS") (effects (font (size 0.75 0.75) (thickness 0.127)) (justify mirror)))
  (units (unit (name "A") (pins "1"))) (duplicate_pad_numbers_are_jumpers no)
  (pad "1" smd circle (at 0 0) (size 1 1) (layers "B.Cu" "B.Mask") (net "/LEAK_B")))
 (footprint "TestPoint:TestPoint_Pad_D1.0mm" (layer "B.Cu") (at 99.55 90.4)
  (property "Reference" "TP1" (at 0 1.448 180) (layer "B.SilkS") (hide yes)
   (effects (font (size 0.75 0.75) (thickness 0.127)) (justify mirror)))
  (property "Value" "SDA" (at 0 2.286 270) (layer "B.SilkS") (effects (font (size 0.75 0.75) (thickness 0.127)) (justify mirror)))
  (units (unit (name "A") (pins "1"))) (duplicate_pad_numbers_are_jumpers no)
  (pad "1" smd circle (at 0 0) (size 1 1) (layers "B.Cu" "B.Mask") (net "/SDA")))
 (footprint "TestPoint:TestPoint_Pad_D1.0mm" (layer "B.Cu") (at 99.55 92.55)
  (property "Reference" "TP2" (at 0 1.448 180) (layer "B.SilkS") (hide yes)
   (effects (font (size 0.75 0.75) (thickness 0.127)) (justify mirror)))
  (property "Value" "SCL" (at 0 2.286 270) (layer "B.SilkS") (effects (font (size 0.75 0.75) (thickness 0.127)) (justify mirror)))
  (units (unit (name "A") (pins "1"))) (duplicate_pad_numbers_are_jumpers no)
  (pad "1" smd circle (at 0 0) (size 1 1) (layers "B.Cu" "B.Mask") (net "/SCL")))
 (gr_arc (start 91.5 90.5) (mid 91.939339 89.439339) (end 93 89) (stroke (width 0.05) (type default)) (layer "Edge.Cuts"))
 (gr_line (start 91.5 100) (end 91.5 90.5) (stroke (width 0.05) (type default)) (layer "Edge.Cuts"))
 (gr_line (start 93 89) (end 107 89) (stroke (width 0.05) (type default)) (layer "Edge.Cuts"))
 (gr_arc (start 107 89) (mid 108.06066 89.439339) (end 108.5 90.5) (stroke (width 0.05) (type default)) (layer "Edge.Cuts"))
 (gr_line (start 108.5 90.5) (end 108.5 100) (stroke (width 0.05) (type default)) (layer "Edge.Cuts"))
 (gr_arc (start 108.5 100) (mid 100 108.5) (end 91.5 100) (stroke (width 0.05) (type default)) (layer "Edge.Cuts"))
 (via (at 105.397 94.769) (size 0.508) (drill 0.254) (layers "F.Cu" "B.Cu") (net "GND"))
 (segment (start 103.81818 95.424286) (end 104 95.606107) (width 0.2) (layer "F.Cu") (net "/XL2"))
 (segment (start 104 95.606107) (end 104 96.031) (width 0.2) (layer "F.Cu") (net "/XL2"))
 (via (at 103.81818 95.424286) (size 0.508) (drill 0.254) (layers "F.Cu" "B.Cu") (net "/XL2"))
 (segment (start 104.816777 95.424212) (end 104.65 95.590989) (width 0.2) (layer "F.Cu") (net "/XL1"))
 (segment (start 104.65 95.590989) (end 104.65 96.031) (width 0.2) (layer "F.Cu") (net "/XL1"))
 (via (at 104.816777 95.424212) (size 0.508) (drill 0.254) (layers "F.Cu" "B.Cu") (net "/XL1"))
 (segment (start 104 93.431) (end 104 92.8132) (width 0.1524) (layer "F.Cu") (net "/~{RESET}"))
 (segment (start 104 92.8132) (end 103.987301 92.8005) (width 0.1524) (layer "F.Cu") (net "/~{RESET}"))
 (via (at 103.987301 92.8005) (size 0.508) (drill 0.254) (layers "F.Cu" "B.Cu") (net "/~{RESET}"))
 (segment (start 102.133001 94.731) (end 101.900001 94.731) (width 0.1524) (layer "F.Cu") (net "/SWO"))
 (segment (start 102.730001 94.134) (end 102.133001 94.731) (width 0.1524) (layer "F.Cu") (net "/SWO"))
 (via (at 102.730001 94.134) (size 0.508) (drill 0.254) (layers "F.Cu" "B.Cu") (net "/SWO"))
 (segment (start 103.350001 95.77) (end 103.350001 96.031) (width 0.2) (layer "F.Cu") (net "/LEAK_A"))
 (segment (start 102.857001 95.277) (end 103.350001 95.77) (width 0.2) (layer "F.Cu") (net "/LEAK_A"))
 (via (at 102.857001 95.277) (size 0.508) (drill 0.254) (layers "F.Cu" "B.Cu") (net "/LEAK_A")))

